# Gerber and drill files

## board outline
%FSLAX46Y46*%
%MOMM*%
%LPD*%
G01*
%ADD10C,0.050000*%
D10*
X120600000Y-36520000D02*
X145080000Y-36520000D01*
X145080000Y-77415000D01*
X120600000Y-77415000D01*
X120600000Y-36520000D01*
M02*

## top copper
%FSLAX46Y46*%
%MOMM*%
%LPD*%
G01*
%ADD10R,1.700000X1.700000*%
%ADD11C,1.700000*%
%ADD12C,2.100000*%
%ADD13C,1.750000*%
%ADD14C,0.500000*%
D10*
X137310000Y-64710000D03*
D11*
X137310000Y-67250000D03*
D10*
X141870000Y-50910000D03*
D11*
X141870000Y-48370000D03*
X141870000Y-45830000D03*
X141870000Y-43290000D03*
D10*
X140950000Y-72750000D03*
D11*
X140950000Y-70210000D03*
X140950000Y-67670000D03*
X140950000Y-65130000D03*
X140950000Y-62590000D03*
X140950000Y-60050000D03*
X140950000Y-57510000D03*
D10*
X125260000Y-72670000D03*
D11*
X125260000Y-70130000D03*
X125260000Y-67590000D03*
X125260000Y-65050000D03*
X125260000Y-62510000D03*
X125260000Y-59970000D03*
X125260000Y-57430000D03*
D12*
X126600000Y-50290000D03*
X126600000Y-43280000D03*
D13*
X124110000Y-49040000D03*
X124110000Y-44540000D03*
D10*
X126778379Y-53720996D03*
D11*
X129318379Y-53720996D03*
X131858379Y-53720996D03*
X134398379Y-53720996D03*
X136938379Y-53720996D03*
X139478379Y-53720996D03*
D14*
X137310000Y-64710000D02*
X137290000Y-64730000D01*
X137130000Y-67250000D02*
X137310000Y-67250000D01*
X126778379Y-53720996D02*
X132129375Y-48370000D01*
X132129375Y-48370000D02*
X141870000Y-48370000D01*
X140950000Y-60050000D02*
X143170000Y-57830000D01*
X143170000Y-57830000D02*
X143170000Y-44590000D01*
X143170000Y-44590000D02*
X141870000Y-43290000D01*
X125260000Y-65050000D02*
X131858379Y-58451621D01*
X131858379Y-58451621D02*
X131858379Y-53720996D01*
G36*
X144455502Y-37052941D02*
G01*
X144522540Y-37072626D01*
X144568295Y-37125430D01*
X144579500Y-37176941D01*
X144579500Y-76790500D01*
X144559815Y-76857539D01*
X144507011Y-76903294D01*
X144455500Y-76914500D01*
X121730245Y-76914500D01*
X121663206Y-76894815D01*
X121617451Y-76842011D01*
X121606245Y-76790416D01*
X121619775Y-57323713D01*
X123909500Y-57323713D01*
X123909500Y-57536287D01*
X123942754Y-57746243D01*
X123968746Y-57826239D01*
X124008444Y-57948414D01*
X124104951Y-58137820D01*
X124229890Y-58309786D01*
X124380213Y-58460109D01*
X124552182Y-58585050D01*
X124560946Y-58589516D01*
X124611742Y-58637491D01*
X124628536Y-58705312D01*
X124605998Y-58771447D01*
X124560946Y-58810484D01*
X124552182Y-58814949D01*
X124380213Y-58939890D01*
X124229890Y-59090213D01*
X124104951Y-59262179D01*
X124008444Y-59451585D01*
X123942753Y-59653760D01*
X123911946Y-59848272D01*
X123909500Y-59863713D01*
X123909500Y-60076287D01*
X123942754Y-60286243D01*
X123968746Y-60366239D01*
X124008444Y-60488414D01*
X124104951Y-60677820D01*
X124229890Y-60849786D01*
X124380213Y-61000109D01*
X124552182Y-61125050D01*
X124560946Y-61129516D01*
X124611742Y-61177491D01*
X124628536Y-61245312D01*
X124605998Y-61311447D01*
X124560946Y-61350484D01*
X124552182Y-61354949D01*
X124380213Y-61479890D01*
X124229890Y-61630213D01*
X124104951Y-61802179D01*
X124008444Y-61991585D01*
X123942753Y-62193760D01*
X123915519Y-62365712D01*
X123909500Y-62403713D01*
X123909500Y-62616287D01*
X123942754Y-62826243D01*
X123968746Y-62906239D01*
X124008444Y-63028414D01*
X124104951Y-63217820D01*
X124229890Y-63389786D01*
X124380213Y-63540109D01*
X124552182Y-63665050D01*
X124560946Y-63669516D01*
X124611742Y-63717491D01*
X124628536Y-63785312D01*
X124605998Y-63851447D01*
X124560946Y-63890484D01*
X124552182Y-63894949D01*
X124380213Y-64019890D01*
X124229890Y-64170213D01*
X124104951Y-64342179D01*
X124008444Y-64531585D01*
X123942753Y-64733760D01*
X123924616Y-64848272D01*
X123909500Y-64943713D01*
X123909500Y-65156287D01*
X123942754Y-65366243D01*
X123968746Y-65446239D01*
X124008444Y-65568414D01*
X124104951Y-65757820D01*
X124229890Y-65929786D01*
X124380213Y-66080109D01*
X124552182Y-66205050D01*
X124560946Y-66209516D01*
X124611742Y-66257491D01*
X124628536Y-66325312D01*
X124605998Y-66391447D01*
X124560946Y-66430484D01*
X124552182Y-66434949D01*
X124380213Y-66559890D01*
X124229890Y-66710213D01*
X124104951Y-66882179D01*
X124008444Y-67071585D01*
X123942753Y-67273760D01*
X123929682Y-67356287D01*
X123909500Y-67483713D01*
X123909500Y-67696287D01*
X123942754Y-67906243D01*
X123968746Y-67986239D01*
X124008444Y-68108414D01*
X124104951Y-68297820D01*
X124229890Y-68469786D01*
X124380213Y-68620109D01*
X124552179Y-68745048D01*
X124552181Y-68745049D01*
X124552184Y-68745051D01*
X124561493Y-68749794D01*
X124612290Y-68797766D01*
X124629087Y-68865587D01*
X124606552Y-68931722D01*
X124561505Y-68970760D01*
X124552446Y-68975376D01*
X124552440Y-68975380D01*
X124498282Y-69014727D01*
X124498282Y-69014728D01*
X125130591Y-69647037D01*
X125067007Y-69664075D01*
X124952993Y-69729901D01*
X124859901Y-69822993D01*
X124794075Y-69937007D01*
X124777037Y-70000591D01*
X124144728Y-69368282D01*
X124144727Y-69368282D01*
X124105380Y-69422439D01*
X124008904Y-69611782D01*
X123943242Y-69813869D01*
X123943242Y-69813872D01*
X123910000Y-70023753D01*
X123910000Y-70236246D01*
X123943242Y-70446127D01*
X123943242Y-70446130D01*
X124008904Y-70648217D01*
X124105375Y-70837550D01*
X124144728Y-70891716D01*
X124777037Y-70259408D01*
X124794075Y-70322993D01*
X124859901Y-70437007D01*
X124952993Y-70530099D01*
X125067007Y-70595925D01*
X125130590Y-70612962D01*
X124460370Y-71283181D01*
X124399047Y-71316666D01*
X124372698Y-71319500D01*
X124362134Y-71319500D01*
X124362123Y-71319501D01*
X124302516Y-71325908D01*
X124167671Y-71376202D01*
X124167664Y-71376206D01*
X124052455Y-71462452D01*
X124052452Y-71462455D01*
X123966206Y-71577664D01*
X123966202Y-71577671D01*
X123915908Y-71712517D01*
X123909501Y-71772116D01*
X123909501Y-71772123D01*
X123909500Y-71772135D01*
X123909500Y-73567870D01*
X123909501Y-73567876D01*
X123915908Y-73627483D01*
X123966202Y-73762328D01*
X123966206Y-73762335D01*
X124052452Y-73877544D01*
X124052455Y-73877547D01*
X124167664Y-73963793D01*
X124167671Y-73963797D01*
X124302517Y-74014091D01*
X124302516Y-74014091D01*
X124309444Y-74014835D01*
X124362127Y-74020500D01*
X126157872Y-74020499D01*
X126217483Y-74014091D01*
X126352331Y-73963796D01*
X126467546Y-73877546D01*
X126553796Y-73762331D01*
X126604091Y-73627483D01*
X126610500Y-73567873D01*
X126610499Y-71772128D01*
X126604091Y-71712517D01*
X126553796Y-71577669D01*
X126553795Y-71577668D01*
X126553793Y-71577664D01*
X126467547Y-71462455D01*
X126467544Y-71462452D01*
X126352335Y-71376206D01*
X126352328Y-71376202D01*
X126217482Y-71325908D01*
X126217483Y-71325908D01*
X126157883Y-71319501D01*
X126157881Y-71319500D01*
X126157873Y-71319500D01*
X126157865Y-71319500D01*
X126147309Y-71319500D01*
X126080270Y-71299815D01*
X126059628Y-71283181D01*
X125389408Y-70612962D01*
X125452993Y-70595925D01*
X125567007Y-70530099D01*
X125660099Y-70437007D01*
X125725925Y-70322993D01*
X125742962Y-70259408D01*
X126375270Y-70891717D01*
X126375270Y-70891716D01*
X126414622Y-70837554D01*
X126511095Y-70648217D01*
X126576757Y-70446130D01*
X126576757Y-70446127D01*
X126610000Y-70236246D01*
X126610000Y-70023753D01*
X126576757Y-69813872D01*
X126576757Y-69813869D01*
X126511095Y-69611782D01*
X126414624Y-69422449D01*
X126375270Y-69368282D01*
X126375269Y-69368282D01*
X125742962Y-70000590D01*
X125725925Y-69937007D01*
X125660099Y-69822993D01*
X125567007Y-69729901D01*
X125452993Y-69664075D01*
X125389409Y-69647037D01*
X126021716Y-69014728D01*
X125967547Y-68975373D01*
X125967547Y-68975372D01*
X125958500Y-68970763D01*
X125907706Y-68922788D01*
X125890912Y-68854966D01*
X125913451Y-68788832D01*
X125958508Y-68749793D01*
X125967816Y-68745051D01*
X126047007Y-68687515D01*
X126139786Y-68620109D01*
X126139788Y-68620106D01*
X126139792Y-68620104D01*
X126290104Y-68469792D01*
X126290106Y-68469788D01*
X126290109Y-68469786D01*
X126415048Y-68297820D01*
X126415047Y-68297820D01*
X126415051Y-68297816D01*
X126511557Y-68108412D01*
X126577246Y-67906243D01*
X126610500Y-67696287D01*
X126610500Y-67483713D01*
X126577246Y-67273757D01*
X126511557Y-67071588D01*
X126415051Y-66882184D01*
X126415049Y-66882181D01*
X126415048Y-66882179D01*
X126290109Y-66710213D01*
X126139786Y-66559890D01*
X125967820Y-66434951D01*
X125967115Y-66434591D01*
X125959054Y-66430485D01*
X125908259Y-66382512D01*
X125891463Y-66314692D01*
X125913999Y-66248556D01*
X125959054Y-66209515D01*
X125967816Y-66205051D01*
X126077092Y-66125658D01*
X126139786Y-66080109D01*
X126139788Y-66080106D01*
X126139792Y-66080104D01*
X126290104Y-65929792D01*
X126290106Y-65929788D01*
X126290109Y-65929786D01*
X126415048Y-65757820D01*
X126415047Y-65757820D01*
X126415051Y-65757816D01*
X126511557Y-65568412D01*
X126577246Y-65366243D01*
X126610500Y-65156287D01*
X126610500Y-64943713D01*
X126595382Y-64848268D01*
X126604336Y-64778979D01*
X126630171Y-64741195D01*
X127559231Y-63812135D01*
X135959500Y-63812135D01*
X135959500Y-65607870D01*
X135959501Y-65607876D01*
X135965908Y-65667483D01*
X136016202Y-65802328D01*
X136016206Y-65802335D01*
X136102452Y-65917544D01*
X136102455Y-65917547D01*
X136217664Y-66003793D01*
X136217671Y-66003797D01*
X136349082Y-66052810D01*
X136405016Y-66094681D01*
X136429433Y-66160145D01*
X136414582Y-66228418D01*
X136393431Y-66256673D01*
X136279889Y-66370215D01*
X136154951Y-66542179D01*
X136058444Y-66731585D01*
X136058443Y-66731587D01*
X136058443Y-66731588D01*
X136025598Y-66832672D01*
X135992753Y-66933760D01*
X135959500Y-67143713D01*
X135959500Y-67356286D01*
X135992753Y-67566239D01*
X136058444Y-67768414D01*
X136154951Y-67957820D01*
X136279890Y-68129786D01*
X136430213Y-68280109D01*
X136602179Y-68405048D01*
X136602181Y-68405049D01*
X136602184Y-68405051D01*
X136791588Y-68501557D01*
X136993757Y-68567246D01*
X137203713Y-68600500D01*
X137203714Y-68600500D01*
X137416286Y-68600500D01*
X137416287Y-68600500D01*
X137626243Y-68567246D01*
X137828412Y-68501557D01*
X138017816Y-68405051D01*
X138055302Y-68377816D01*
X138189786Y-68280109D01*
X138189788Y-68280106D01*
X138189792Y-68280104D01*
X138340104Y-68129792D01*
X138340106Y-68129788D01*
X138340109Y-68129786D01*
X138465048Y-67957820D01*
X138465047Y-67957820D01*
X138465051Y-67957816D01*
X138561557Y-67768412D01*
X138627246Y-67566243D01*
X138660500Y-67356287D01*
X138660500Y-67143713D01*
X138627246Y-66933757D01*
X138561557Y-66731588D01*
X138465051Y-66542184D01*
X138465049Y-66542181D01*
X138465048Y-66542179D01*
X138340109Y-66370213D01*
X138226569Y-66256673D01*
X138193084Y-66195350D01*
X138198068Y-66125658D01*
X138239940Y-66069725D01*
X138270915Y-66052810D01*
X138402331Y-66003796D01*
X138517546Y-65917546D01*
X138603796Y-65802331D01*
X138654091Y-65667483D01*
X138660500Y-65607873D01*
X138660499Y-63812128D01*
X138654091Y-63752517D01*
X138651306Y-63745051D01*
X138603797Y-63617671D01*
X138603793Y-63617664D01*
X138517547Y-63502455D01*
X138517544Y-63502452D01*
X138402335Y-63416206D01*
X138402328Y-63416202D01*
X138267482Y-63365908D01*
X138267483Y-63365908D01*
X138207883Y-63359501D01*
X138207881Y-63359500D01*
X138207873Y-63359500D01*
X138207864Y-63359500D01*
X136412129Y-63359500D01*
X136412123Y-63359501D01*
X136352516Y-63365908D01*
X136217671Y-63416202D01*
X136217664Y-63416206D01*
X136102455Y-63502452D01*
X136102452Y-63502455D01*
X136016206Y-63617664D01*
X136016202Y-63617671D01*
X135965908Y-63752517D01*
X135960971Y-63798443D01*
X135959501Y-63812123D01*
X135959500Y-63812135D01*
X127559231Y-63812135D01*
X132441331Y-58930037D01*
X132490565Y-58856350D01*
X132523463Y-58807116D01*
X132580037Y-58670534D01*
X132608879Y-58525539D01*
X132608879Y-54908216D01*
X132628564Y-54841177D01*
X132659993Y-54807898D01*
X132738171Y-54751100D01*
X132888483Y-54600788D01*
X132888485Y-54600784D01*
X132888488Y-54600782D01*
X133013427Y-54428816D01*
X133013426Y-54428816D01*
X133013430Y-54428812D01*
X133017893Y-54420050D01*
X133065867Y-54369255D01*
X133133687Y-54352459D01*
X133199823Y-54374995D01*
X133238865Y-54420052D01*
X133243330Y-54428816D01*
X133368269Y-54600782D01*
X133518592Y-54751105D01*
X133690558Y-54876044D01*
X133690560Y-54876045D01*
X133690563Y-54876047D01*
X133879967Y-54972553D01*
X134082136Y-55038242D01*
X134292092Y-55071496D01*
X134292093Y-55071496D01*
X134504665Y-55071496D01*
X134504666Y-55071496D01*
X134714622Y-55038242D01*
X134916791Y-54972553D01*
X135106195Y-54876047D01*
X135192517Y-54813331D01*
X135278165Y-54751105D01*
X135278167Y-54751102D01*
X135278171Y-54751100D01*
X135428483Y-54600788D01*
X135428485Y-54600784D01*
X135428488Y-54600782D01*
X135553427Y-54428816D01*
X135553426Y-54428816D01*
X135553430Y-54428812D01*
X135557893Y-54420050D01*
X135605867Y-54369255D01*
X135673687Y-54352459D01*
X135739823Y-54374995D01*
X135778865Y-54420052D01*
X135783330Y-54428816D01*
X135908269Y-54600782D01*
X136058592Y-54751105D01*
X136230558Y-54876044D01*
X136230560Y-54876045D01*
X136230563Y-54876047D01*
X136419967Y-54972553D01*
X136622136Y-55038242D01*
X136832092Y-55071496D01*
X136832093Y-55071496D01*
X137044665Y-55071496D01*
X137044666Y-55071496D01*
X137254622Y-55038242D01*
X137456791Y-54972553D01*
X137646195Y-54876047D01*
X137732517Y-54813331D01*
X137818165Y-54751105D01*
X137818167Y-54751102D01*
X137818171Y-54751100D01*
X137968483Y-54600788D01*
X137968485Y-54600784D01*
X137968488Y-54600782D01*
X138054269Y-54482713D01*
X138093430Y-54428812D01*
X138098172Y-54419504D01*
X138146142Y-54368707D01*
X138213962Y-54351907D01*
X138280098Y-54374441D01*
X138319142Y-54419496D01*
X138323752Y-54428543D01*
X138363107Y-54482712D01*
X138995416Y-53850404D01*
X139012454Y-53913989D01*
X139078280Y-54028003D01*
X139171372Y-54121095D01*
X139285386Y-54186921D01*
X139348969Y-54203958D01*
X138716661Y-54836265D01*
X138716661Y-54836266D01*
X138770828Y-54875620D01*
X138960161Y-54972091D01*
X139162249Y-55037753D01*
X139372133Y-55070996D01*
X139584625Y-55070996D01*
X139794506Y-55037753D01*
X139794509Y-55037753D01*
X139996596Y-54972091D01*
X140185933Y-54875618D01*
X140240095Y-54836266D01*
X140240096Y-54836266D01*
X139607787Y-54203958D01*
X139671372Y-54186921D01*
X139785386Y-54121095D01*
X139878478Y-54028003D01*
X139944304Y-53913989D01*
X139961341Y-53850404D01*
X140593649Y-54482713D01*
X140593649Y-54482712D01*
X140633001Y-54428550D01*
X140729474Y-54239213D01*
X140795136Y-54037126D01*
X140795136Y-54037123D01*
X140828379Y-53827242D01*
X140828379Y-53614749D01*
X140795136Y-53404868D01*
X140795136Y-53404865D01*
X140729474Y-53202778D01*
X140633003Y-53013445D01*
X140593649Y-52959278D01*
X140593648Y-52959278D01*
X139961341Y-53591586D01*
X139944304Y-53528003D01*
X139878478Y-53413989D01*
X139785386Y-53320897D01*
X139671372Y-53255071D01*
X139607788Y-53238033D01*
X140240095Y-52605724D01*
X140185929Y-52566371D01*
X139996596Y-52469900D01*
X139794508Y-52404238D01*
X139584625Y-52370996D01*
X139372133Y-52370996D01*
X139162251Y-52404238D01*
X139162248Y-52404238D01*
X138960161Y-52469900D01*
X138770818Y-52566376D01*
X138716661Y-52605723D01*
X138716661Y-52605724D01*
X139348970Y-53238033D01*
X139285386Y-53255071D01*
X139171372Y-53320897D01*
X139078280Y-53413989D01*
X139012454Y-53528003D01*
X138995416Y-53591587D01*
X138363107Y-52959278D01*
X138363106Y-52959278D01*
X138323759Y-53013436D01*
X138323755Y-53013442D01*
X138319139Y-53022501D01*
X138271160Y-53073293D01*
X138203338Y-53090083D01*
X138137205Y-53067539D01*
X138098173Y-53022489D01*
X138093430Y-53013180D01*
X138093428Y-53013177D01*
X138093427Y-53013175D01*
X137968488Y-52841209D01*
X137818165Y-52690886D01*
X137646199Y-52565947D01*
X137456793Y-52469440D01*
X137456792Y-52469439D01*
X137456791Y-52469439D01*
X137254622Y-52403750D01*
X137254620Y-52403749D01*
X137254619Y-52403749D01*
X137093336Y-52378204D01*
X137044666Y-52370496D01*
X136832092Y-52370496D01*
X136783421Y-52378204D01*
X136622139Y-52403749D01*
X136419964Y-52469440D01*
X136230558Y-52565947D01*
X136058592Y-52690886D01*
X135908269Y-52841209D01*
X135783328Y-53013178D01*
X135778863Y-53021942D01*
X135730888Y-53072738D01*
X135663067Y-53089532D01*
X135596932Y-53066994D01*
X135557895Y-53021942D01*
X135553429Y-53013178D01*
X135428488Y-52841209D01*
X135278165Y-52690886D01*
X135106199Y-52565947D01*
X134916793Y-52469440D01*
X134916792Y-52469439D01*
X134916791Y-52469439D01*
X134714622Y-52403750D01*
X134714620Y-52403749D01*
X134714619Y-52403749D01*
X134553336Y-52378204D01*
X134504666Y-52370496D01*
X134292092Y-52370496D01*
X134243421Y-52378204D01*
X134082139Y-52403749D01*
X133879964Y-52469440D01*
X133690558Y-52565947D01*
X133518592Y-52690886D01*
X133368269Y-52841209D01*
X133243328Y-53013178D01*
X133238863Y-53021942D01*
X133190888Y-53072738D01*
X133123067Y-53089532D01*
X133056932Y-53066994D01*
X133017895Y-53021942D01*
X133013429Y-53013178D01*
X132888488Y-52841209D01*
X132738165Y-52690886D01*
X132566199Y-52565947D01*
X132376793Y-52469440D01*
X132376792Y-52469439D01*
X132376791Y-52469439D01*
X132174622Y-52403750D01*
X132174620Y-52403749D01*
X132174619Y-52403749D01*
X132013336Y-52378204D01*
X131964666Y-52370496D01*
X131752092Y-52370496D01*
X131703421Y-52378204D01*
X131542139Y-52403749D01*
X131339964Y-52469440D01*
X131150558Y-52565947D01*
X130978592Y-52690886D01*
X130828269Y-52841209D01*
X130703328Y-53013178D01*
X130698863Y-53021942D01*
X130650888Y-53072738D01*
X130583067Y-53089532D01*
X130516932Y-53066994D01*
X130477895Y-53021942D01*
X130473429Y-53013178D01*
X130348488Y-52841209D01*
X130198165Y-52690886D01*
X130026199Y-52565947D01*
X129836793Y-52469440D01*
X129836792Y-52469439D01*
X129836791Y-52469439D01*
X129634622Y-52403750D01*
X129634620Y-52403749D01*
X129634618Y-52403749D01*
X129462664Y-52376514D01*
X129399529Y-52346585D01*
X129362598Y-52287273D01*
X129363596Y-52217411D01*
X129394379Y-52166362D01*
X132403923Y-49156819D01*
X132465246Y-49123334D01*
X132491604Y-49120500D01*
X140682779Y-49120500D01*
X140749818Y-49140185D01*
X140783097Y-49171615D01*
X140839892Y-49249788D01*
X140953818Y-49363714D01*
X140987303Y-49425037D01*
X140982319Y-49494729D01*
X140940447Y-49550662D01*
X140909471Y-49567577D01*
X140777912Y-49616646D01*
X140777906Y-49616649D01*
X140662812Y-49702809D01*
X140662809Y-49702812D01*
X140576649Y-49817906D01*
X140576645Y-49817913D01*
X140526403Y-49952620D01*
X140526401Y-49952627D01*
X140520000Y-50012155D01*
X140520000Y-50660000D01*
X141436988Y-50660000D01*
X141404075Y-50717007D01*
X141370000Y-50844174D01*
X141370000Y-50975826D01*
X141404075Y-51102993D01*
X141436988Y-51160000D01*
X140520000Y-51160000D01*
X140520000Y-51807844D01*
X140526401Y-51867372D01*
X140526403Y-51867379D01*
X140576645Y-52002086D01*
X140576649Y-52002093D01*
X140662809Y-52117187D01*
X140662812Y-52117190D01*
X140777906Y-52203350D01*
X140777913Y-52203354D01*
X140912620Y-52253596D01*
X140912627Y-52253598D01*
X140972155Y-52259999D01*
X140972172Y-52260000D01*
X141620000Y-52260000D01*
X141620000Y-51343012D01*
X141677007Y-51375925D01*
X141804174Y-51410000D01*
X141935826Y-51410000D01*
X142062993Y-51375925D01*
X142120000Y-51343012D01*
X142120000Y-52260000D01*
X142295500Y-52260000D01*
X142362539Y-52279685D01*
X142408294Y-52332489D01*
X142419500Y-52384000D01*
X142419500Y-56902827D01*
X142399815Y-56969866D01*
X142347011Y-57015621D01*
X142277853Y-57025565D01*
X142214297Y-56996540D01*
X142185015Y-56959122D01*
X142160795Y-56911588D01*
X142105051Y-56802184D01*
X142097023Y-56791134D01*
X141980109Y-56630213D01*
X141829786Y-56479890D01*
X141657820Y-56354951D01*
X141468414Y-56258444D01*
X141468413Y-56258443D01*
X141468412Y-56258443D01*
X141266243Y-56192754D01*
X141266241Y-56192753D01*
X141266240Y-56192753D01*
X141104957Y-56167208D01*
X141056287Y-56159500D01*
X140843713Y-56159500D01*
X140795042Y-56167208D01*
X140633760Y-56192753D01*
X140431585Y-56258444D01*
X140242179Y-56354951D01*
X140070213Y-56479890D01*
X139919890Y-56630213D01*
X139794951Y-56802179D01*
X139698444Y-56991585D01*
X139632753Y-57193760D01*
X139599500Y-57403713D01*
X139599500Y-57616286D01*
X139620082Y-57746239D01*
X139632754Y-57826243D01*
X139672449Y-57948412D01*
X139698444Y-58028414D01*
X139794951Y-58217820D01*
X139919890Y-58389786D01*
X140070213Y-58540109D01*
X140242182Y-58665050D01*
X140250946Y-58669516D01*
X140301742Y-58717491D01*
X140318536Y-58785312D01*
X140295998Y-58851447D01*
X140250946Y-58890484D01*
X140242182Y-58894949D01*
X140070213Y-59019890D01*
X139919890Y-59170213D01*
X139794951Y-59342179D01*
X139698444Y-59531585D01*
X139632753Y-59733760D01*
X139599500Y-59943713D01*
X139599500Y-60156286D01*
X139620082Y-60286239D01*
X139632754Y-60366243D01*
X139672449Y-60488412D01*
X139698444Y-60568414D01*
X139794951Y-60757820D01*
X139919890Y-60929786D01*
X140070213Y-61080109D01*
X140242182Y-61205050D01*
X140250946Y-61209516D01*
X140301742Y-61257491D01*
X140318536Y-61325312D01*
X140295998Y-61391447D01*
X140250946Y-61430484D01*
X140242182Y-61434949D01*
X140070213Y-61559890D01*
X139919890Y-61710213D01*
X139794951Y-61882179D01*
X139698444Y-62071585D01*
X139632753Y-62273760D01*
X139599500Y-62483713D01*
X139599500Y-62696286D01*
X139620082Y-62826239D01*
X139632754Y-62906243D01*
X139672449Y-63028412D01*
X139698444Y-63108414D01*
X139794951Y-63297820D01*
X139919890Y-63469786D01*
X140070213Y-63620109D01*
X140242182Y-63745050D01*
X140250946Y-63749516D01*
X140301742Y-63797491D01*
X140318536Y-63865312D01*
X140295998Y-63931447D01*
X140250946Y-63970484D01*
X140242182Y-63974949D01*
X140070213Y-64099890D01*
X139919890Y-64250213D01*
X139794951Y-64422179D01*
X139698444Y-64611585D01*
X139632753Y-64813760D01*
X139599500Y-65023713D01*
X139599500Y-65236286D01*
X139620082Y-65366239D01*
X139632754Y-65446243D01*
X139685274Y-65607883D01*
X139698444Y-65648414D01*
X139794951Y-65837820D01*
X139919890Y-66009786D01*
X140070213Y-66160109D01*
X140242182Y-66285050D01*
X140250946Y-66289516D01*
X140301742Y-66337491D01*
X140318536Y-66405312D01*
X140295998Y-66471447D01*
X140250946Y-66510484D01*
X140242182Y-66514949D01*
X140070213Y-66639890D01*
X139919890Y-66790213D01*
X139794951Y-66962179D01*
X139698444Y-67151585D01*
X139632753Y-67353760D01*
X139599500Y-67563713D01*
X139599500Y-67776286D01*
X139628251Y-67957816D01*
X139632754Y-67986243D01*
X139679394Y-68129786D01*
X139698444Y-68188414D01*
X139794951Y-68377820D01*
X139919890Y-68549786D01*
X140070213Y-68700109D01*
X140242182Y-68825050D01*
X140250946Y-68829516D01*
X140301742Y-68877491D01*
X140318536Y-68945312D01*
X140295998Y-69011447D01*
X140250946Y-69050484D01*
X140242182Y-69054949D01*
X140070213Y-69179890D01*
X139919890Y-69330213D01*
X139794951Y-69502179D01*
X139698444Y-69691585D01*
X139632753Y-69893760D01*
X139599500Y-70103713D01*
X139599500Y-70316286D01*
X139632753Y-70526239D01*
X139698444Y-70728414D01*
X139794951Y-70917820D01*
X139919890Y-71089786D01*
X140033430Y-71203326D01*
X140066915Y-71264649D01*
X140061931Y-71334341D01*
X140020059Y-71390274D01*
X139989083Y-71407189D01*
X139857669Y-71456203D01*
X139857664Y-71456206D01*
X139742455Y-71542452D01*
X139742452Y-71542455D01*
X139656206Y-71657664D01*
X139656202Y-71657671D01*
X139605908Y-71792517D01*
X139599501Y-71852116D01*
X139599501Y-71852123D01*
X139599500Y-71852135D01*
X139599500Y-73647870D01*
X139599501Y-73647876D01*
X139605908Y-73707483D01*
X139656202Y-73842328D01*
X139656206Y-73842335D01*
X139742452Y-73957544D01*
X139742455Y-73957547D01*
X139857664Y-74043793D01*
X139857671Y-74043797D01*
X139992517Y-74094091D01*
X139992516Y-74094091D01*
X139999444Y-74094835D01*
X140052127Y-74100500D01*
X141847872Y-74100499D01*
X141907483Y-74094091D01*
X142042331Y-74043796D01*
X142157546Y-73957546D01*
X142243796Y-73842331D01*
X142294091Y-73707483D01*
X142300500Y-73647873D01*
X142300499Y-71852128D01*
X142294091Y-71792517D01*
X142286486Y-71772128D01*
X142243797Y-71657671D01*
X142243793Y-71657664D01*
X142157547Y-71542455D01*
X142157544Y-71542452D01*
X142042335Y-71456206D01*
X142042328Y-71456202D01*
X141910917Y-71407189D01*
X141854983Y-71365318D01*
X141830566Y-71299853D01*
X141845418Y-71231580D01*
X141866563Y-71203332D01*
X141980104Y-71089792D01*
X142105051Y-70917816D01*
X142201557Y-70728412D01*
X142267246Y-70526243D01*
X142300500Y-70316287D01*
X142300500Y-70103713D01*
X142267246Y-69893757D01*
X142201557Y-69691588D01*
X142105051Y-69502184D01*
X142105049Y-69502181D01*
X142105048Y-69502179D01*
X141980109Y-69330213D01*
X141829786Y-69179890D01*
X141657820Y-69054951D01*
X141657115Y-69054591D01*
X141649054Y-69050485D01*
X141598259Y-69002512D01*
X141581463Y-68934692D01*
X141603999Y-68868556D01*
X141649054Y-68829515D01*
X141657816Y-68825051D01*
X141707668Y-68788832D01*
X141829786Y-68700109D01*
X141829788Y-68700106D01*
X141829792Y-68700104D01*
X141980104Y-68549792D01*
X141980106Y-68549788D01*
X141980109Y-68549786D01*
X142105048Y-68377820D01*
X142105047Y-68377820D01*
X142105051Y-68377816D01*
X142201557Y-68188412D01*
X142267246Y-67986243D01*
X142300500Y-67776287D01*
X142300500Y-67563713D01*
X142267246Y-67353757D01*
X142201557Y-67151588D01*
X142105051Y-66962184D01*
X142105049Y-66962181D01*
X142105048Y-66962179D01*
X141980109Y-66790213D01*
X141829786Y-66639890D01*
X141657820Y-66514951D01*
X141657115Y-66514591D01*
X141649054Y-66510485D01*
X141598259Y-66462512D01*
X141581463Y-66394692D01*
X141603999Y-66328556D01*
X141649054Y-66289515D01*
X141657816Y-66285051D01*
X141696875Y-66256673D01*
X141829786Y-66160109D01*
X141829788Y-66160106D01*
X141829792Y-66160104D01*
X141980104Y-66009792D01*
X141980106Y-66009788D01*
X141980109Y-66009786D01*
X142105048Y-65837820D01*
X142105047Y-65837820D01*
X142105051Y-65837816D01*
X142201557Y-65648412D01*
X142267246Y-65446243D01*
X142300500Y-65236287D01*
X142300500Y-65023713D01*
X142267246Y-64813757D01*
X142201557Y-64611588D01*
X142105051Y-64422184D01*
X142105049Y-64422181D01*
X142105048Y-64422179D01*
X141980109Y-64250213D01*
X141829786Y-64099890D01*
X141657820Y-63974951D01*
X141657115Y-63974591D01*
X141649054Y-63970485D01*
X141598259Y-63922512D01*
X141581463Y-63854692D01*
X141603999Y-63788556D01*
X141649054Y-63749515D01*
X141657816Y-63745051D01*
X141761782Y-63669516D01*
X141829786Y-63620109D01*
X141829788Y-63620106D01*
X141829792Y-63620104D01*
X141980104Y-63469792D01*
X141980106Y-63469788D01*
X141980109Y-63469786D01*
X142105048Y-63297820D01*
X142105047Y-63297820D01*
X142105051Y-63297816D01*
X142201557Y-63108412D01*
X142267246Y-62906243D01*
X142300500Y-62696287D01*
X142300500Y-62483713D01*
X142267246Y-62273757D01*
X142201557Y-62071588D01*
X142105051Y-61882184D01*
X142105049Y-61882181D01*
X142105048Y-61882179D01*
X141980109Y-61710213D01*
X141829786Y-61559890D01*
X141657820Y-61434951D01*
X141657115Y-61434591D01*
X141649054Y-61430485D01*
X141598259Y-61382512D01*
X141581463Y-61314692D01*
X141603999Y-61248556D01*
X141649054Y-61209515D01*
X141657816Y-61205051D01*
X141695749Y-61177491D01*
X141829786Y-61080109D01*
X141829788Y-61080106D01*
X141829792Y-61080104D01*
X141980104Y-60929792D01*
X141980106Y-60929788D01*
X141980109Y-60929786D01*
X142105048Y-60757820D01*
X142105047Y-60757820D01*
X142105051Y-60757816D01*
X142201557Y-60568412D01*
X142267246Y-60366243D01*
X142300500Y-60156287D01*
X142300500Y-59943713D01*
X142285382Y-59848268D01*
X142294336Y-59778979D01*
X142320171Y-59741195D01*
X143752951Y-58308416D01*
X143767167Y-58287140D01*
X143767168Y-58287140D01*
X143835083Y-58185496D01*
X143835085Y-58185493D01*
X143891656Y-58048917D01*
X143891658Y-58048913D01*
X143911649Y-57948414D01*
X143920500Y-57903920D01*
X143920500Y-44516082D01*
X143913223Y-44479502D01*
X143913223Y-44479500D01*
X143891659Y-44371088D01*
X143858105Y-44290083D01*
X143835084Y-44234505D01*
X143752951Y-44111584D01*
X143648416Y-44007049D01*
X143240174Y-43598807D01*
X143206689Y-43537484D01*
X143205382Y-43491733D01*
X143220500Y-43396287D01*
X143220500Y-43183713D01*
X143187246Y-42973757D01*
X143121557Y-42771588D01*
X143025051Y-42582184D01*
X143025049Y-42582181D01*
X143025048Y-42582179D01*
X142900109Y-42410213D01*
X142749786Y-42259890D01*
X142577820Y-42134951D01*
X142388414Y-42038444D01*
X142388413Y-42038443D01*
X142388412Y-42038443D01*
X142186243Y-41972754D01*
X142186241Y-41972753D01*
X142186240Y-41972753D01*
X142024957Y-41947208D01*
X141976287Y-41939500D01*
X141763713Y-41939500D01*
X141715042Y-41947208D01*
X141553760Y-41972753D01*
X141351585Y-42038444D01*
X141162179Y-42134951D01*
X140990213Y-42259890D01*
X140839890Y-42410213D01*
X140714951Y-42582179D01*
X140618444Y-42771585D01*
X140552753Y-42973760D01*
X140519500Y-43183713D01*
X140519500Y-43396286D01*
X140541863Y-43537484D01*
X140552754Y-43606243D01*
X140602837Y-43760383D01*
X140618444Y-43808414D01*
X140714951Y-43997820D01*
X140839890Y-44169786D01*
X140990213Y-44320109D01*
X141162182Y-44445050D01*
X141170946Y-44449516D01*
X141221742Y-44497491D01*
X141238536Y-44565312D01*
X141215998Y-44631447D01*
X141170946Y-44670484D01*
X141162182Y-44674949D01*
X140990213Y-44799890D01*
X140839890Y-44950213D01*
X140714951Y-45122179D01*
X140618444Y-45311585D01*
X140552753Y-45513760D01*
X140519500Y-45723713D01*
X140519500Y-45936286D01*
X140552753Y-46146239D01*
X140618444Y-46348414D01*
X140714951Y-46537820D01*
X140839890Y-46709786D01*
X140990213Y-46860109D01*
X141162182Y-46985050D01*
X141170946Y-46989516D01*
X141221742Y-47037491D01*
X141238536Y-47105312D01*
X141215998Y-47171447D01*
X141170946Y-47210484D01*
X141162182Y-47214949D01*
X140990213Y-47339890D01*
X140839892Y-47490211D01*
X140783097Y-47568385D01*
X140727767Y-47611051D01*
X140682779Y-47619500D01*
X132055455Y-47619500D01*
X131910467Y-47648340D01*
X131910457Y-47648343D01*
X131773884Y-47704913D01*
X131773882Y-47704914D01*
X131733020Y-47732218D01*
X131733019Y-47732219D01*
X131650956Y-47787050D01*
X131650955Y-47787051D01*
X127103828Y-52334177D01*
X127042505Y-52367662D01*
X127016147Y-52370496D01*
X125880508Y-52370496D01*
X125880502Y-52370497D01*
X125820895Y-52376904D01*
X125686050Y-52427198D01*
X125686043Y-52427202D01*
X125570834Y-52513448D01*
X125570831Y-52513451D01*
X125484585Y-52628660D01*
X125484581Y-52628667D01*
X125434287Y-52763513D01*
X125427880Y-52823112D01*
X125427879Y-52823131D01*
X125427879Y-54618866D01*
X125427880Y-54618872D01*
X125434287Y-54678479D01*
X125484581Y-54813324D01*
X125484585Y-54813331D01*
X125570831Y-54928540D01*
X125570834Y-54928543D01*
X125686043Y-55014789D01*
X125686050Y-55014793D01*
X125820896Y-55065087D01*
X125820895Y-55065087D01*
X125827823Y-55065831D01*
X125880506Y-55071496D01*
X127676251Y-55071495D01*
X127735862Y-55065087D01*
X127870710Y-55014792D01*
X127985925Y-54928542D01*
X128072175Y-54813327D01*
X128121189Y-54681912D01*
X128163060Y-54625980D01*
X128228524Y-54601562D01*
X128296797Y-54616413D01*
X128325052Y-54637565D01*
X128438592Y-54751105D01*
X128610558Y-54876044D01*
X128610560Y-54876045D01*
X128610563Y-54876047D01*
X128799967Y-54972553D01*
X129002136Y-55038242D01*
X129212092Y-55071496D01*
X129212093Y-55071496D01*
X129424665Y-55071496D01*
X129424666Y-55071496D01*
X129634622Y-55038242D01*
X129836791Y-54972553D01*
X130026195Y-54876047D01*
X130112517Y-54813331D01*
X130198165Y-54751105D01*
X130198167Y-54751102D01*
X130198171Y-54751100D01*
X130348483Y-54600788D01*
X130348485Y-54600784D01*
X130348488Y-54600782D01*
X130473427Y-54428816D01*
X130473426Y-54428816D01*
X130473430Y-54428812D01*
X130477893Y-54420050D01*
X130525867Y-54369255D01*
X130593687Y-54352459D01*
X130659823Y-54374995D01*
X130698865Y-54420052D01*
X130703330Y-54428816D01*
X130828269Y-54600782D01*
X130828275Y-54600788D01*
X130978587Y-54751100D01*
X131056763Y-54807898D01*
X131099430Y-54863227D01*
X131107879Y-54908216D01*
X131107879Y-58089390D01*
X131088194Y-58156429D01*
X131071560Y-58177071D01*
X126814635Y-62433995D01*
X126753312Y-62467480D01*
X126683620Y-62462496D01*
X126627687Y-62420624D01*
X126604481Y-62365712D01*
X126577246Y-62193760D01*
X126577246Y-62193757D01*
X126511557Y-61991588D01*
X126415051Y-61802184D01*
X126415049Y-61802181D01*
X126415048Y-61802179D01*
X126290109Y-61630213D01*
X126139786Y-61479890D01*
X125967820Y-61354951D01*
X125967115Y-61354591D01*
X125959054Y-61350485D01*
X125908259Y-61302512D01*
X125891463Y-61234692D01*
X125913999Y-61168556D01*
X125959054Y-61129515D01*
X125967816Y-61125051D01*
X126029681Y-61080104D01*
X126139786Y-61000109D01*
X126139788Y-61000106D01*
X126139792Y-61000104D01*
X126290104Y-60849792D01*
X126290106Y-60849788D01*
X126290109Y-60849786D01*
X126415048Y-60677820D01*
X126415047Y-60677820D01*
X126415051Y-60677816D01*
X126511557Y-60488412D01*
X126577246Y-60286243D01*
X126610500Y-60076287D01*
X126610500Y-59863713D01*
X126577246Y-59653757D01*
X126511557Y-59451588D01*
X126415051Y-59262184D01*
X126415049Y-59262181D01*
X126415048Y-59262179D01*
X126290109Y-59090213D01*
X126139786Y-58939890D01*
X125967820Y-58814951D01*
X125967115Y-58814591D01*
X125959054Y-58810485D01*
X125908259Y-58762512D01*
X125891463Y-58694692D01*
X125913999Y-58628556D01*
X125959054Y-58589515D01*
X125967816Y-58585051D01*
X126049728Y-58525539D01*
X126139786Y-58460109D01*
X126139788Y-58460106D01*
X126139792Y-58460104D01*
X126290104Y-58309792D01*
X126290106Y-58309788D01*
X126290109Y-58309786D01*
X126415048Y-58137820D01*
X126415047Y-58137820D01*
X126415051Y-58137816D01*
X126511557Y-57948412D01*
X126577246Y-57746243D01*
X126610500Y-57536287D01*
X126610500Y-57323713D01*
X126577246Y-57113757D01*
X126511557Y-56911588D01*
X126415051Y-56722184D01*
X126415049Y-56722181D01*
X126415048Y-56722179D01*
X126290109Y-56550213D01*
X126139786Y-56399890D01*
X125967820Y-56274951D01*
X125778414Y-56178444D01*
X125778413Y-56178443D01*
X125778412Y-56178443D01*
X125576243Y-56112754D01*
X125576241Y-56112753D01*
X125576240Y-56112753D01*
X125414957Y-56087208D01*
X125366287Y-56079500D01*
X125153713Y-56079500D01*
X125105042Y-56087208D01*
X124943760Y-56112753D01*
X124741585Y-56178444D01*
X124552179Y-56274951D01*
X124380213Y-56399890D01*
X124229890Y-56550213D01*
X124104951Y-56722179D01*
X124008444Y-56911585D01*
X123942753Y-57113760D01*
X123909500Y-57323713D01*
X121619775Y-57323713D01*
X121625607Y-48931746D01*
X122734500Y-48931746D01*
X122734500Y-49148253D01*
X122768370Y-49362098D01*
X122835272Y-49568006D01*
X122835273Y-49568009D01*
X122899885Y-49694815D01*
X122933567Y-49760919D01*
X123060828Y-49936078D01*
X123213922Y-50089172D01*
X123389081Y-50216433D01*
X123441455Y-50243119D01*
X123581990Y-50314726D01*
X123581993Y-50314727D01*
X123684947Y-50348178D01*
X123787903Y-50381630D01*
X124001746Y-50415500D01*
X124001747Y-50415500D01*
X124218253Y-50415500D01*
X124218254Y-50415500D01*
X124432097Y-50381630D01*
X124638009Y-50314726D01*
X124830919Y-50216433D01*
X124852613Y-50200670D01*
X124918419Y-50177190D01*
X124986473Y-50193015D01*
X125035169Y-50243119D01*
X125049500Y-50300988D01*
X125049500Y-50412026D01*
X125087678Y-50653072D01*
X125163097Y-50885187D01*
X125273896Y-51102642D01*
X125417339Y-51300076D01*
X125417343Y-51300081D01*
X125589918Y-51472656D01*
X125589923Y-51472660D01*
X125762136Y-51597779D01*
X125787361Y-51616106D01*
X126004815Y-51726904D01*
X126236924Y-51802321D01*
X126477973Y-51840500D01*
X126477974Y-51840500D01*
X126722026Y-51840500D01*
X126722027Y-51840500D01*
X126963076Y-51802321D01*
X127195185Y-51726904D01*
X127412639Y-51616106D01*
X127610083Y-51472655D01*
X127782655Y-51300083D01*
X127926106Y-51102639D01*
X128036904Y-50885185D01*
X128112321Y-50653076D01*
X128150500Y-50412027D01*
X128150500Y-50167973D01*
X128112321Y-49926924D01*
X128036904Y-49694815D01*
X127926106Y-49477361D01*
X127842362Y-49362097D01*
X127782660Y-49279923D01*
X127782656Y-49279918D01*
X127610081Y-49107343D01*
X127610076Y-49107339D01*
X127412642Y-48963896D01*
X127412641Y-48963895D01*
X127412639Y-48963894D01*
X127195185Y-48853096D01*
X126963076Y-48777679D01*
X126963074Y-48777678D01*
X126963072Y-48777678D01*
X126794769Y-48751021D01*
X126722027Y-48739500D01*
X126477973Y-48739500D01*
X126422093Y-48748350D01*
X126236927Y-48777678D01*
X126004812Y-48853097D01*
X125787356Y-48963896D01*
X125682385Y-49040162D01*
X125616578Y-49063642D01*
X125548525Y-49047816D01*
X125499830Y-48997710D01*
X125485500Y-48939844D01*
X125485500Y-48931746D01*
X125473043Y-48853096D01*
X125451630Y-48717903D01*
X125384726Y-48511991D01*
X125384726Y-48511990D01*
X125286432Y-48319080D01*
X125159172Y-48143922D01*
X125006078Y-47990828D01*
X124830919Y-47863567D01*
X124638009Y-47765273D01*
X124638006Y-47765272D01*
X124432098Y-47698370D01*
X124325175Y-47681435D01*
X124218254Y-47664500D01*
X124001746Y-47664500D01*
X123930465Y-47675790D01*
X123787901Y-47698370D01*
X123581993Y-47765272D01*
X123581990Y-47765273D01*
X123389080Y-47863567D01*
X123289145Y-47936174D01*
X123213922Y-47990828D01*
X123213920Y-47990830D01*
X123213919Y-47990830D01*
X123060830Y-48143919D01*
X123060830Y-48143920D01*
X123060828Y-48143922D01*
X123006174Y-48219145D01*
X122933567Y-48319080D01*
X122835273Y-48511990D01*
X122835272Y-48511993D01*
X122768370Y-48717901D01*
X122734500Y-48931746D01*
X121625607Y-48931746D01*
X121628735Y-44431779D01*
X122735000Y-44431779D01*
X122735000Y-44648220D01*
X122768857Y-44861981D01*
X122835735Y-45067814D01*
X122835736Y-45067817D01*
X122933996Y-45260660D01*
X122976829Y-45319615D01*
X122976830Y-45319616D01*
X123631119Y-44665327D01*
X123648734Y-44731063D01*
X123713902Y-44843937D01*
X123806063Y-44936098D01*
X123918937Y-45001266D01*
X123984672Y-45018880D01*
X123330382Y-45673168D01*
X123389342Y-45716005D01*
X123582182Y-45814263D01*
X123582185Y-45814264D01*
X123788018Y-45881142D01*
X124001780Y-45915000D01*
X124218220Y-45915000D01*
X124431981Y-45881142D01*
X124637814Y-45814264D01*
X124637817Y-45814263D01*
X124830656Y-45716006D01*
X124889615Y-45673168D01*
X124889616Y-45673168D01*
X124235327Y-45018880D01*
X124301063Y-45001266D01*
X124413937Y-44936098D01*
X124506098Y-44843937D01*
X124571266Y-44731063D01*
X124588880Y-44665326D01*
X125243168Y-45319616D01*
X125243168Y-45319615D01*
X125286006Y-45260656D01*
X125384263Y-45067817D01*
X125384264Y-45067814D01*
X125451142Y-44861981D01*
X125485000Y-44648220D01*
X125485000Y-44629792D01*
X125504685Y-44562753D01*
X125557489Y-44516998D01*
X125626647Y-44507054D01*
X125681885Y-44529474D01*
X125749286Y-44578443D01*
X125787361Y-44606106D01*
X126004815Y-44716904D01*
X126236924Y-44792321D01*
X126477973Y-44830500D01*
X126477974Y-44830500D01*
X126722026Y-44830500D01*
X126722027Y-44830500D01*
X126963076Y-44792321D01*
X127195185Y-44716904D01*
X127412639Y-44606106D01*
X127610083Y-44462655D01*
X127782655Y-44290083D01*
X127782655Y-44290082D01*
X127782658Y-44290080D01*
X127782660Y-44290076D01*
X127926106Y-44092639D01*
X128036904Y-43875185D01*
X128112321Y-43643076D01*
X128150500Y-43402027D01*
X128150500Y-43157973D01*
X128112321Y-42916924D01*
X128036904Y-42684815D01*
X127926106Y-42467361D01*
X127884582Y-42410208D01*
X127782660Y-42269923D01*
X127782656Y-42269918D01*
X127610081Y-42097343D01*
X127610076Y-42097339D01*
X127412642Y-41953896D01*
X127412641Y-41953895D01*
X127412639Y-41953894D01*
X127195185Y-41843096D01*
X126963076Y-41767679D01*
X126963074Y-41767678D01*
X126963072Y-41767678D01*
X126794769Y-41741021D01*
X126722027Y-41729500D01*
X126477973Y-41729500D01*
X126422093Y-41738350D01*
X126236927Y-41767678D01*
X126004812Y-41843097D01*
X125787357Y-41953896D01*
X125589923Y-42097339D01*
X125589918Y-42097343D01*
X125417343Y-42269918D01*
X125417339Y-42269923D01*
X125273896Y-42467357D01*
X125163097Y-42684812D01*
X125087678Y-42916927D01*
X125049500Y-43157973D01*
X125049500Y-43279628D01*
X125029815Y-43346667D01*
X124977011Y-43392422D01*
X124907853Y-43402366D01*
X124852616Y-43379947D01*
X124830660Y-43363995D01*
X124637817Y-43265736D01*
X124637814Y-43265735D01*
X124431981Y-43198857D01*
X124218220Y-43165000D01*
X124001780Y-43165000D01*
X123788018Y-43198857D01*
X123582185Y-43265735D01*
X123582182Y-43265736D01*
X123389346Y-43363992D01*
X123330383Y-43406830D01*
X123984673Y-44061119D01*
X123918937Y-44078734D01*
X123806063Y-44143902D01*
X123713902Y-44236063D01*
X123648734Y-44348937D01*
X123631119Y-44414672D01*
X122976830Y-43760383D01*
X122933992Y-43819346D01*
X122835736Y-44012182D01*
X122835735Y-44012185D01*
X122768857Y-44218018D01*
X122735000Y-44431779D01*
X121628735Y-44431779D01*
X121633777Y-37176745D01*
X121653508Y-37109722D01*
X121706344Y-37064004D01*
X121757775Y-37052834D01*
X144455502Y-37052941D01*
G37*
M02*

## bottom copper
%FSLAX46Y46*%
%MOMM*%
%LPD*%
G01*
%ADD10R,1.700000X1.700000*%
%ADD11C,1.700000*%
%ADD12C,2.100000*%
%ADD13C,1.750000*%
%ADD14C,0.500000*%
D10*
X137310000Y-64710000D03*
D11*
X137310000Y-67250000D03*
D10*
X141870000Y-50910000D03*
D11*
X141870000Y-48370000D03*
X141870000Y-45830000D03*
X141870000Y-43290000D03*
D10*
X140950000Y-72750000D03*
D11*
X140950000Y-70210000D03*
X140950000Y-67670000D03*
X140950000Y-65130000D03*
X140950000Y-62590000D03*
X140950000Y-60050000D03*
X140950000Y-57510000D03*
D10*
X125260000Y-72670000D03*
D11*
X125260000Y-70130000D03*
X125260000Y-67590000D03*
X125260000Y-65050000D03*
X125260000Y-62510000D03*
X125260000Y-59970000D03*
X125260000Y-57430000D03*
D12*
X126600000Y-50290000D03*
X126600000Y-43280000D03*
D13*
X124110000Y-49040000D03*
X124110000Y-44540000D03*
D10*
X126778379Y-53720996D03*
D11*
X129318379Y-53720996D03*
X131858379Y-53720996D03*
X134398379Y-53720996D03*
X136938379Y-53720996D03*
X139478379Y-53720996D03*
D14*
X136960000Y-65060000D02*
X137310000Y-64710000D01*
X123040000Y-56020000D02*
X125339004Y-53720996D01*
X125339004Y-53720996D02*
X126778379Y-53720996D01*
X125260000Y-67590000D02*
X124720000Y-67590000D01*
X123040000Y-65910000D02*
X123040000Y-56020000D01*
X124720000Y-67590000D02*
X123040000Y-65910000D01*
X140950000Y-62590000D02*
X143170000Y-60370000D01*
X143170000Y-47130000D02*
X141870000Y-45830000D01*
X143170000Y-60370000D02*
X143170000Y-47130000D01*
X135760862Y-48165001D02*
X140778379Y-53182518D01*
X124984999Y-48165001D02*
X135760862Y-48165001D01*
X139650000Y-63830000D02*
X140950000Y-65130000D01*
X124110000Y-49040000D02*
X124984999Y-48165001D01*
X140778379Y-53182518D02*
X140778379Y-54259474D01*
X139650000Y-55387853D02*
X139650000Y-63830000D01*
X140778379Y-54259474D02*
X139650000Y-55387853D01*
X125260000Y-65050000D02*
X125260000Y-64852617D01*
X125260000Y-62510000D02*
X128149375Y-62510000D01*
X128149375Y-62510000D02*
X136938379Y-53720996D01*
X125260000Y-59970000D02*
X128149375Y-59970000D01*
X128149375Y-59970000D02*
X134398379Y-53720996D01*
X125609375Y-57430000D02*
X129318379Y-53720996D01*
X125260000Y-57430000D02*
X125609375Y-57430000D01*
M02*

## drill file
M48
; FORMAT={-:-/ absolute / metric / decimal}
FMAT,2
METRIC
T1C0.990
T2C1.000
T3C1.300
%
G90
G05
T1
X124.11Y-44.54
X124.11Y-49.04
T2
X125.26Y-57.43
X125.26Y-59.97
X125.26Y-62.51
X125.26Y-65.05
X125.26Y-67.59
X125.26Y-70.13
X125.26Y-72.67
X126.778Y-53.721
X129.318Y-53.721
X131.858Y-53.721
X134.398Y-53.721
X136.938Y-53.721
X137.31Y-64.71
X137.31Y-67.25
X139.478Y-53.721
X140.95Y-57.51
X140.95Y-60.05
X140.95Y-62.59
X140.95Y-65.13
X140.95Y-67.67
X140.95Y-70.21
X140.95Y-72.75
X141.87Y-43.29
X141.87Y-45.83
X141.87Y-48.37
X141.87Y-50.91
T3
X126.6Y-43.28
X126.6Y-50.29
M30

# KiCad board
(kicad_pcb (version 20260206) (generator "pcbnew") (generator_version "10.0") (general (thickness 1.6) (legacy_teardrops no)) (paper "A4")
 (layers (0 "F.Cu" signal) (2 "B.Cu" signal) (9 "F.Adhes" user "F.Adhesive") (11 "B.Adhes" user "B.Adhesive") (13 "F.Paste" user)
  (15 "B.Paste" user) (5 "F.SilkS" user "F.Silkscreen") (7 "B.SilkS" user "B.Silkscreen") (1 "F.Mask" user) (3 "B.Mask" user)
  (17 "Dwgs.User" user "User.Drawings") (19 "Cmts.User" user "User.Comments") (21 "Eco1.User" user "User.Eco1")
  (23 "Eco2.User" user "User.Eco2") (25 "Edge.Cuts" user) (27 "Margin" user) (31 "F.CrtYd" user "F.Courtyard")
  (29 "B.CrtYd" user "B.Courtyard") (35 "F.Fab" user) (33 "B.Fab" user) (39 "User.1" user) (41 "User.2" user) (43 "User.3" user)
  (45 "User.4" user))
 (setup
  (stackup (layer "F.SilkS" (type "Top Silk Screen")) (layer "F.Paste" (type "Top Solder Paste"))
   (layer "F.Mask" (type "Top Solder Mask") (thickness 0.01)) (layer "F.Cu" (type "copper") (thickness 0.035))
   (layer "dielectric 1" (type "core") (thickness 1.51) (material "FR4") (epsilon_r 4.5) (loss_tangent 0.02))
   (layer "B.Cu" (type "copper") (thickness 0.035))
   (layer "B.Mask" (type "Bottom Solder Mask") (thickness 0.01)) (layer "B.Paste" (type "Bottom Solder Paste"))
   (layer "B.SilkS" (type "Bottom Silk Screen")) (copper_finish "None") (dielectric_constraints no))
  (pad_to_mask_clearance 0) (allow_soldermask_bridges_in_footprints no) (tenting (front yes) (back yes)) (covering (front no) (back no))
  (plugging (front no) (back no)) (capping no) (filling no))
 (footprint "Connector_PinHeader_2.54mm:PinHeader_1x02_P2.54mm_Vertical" (layer "F.Cu") (at 137.31 64.71)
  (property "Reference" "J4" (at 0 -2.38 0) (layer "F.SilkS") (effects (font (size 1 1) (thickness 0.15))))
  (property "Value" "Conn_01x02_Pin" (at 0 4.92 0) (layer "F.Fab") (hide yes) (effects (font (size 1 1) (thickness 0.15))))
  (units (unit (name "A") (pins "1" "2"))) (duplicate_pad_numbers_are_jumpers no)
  (pad "1" thru_hole rect (at 0 0) (size 1.7 1.7) (drill 1) (layers "*.Cu" "*.Mask") (remove_unused_layers no) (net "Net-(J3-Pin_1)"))
  (pad "2" thru_hole circle (at 0 2.54) (size 1.7 1.7) (drill 1) (layers "*.Cu" "*.Mask") (remove_unused_layers no) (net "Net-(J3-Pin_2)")))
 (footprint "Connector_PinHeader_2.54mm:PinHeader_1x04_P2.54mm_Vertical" (layer "F.Cu") (at 141.87 50.91 180)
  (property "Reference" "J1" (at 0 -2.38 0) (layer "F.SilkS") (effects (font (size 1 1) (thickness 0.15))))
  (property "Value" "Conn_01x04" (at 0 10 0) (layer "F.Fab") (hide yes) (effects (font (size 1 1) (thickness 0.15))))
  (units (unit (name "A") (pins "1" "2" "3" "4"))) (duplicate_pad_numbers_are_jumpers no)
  (pad "1" thru_hole rect (at 0 0 180) (size 1.7 1.7) (drill 1) (layers "*.Cu" "*.Mask") (remove_unused_layers no) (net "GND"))
  (pad "2" thru_hole circle (at 0 2.54 180) (size 1.7 1.7) (drill 1) (layers "*.Cu" "*.Mask") (remove_unused_layers no) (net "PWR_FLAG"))
  (pad "3" thru_hole circle (at 0 5.08 180) (size 1.7 1.7) (drill 1) (layers "*.Cu" "*.Mask") (remove_unused_layers no)
   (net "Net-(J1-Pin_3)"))
  (pad "4" thru_hole circle (at 0 7.62 180) (size 1.7 1.7) (drill 1) (layers "*.Cu" "*.Mask") (remove_unused_layers no)
   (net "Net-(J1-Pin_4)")))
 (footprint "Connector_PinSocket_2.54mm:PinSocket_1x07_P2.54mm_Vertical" (layer "F.Cu") (at 140.95 72.75 180)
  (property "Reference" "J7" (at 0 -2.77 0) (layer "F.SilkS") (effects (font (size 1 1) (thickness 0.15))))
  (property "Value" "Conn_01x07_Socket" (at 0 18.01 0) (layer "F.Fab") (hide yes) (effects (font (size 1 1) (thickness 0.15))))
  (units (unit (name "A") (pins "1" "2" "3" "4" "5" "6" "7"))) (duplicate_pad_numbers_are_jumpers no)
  (pad "1" thru_hole rect (at 0 0 180) (size 1.7 1.7) (drill 1) (layers "*.Cu" "*.Mask") (remove_unused_layers no) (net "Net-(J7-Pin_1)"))
  (pad "2" thru_hole circle (at 0 2.54 180) (size 1.7 1.7) (drill 1) (layers "*.Cu" "*.Mask") (remove_unused_layers no)
   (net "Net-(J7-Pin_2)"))
  (pad "3" thru_hole circle (at 0 5.08 180) (size 1.7 1.7) (drill 1) (layers "*.Cu" "*.Mask") (remove_unused_layers no)
   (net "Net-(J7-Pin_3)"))
  (pad "4" thru_hole circle (at 0 7.62 180) (size 1.7 1.7) (drill 1) (layers "*.Cu" "*.Mask") (remove_unused_layers no)
   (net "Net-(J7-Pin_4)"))
  (pad "5" thru_hole circle (at 0 10.16 180) (size 1.7 1.7) (drill 1) (layers "*.Cu" "*.Mask") (remove_unused_layers no)
   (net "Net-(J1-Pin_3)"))
  (pad "6" thru_hole circle (at 0 12.7 180) (size 1.7 1.7) (drill 1) (layers "*.Cu" "*.Mask") (remove_unused_layers no)
   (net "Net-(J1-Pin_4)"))
  (pad "7" thru_hole circle (at 0 15.24 180) (size 1.7 1.7) (drill 1) (layers "*.Cu" "*.Mask") (remove_unused_layers no)
   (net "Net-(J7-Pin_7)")))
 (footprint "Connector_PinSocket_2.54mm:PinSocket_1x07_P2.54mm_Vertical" (layer "F.Cu") (at 125.26 72.67 180)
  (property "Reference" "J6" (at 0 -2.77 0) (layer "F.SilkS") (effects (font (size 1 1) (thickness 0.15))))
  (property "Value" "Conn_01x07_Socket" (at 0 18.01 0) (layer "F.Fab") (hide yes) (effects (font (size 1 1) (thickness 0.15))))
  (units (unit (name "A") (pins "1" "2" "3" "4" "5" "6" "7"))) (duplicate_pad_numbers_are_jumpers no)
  (pad "1" thru_hole rect (at 0 0 180) (size 1.7 1.7) (drill 1) (layers "*.Cu" "*.Mask") (remove_unused_layers no) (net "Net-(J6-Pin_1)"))
  (pad "2" thru_hole circle (at 0 2.54 180) (size 1.7 1.7) (drill 1) (layers "*.Cu" "*.Mask") (remove_unused_layers no) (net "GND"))
  (pad "3" thru_hole circle (at 0 5.08 180) (size 1.7 1.7) (drill 1) (layers "*.Cu" "*.Mask") (remove_unused_layers no) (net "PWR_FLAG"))
  (pad "4" thru_hole circle (at 0 7.62 180) (size 1.7 1.7) (drill 1) (layers "*.Cu" "*.Mask") (remove_unused_layers no)
   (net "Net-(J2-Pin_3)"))
  (pad "5" thru_hole circle (at 0 10.16 180) (size 1.7 1.7) (drill 1) (layers "*.Cu" "*.Mask") (remove_unused_layers no)
   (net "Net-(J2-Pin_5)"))
  (pad "6" thru_hole circle (at 0 12.7 180) (size 1.7 1.7) (drill 1) (layers "*.Cu" "*.Mask") (remove_unused_layers no)
   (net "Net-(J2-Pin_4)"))
  (pad "7" thru_hole circle (at 0 15.24 180) (size 1.7 1.7) (drill 1) (layers "*.Cu" "*.Mask") (remove_unused_layers no)
   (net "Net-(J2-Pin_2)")))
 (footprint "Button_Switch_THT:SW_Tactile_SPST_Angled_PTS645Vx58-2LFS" (layer "F.Cu") (at 124.11 49.04 90)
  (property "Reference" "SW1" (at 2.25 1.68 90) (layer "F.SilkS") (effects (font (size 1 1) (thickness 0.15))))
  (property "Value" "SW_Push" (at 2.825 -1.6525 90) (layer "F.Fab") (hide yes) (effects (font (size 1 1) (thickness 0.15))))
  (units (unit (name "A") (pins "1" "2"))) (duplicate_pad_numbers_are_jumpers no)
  (pad "" thru_hole circle (at -1.25 2.49 90) (size 2.1 2.1) (drill 1.3) (layers "*.Cu" "*.Mask") (remove_unused_layers no))
  (pad "" thru_hole circle (at 5.76 2.49 90) (size 2.1 2.1) (drill 1.3) (layers "*.Cu" "*.Mask") (remove_unused_layers no))
  (pad "1" thru_hole circle (at 0 0 90) (size 1.75 1.75) (drill 0.99) (layers "*.Cu" "*.Mask") (remove_unused_layers no)
   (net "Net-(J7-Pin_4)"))
  (pad "2" thru_hole circle (at 4.5 0 90) (size 1.75 1.75) (drill 0.99) (layers "*.Cu" "*.Mask") (remove_unused_layers no) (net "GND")))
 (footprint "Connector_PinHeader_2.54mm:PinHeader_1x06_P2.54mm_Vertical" (layer "B.Cu") (at 126.778379 53.720996 -90)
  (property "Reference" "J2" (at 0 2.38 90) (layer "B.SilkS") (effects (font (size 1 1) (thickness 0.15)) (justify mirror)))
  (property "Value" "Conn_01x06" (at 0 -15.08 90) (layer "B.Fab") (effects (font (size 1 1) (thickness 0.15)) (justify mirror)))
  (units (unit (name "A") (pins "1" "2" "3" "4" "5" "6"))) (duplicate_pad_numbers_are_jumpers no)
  (pad "1" thru_hole rect (at 0 0 270) (size 1.7 1.7) (drill 1) (layers "*.Cu" "*.Mask") (remove_unused_layers no) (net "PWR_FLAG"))
  (pad "2" thru_hole circle (at 0 -2.54 270) (size 1.7 1.7) (drill 1) (layers "*.Cu" "*.Mask") (remove_unused_layers no)
   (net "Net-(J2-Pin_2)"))
  (pad "3" thru_hole circle (at 0 -5.08 270) (size 1.7 1.7) (drill 1) (layers "*.Cu" "*.Mask") (remove_unused_layers no)
   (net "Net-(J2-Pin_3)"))
  (pad "4" thru_hole circle (at 0 -7.62 270) (size 1.7 1.7) (drill 1) (layers "*.Cu" "*.Mask") (remove_unused_layers no)
   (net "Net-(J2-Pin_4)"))
  (pad "5" thru_hole circle (at 0 -10.16 270) (size 1.7 1.7) (drill 1) (layers "*.Cu" "*.Mask") (remove_unused_layers no)
   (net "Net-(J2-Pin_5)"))
  (pad "6" thru_hole circle (at 0 -12.7 270) (size 1.7 1.7) (drill 1) (layers "*.Cu" "*.Mask") (remove_unused_layers no) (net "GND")))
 (gr_rect (start 120.6 36.52) (end 145.08 77.415) (stroke (width 0.05) (type default)) (fill no) (layer "Edge.Cuts"))
 (segment (start 137.31 64.71) (end 137.29 64.73) (width 0.5) (layer "F.Cu") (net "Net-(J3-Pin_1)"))
 (segment (start 136.96 65.06) (end 137.31 64.71) (width 0.5) (layer "B.Cu") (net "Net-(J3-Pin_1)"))
 (segment (start 137.13 67.25) (end 137.31 67.25) (width 0.5) (layer "F.Cu") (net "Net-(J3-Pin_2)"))
 (segment (start 126.778379 53.720996) (end 132.129375 48.37) (width 0.5) (layer "F.Cu") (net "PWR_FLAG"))
 (segment (start 132.129375 48.37) (end 141.87 48.37) (width 0.5) (layer "F.Cu") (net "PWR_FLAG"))
 (segment (start 123.04 56.02) (end 125.339004 53.720996) (width 0.5) (layer "B.Cu") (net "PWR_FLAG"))
 (segment (start 125.339004 53.720996) (end 126.778379 53.720996) (width 0.5) (layer "B.Cu") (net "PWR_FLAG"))
 (segment (start 125.26 67.59) (end 124.72 67.59) (width 0.5) (layer "B.Cu") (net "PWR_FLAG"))
 (segment (start 123.04 65.91) (end 123.04 56.02) (width 0.5) (layer "B.Cu") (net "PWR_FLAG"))
 (segment (start 124.72 67.59) (end 123.04 65.91) (width 0.5) (layer "B.Cu") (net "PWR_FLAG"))
 (segment (start 140.95 62.59) (end 143.17 60.37) (width 0.5) (layer "B.Cu") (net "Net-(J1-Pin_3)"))
 (segment (start 143.17 47.13) (end 141.87 45.83) (width 0.5) (layer "B.Cu") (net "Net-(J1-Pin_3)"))
 (segment (start 143.17 60.37) (end 143.17 47.13) (width 0.5) (layer "B.Cu") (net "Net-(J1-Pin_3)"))
 (segment (start 140.95 60.05) (end 143.17 57.83) (width 0.5) (layer "F.Cu") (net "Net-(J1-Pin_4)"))
 (segment (start 143.17 57.83) (end 143.17 44.59) (width 0.5) (layer "F.Cu") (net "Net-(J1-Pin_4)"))
 (segment (start 143.17 44.59) (end 141.87 43.29) (width 0.5) (layer "F.Cu") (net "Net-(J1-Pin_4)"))
 (segment (start 135.760862 48.165001) (end 140.778379 53.182518) (width 0.5) (layer "B.Cu") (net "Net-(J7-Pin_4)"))
 (segment (start 124.984999 48.165001) (end 135.760862 48.165001) (width 0.5) (layer "B.Cu") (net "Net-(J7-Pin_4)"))
 (segment (start 139.65 63.83) (end 140.95 65.13) (width 0.5) (layer "B.Cu") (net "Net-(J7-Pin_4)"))
 (segment (start 124.11 49.04) (end 124.984999 48.165001) (width 0.5) (layer "B.Cu") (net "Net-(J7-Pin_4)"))
 (segment (start 140.778379 53.182518) (end 140.778379 54.259474) (width 0.5) (layer "B.Cu") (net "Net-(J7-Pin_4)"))
 (segment (start 139.65 55.387853) (end 139.65 63.83) (width 0.5) (layer "B.Cu") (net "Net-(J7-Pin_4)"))
 (segment (start 140.778379 54.259474) (end 139.65 55.387853) (width 0.5) (layer "B.Cu") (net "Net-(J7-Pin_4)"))
 (segment (start 125.26 65.05) (end 131.858379 58.451621) (width 0.5) (layer "F.Cu") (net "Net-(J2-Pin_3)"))
 (segment (start 131.858379 58.451621) (end 131.858379 53.720996) (width 0.5) (layer "F.Cu") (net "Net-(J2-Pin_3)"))
 (segment (start 125.26 65.05) (end 125.26 64.852617) (width 0.5) (layer "B.Cu") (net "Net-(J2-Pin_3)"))
 (segment (start 125.26 62.51) (end 128.149375 62.51) (width 0.5) (layer "B.Cu") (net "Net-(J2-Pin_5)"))
 (segment (start 128.149375 62.51) (end 136.938379 53.720996) (width 0.5) (layer "B.Cu") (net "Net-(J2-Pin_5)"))
 (segment (start 125.26 59.97) (end 128.149375 59.97) (width 0.5) (layer "B.Cu") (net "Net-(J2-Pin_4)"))
 (segment (start 128.149375 59.97) (end 134.398379 53.720996) (width 0.5) (layer "B.Cu") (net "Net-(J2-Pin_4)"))
 (segment (start 125.609375 57.43) (end 129.318379 53.720996) (width 0.5) (layer "B.Cu") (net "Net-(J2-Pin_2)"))
 (segment (start 125.26 57.43) (end 125.609375 57.43) (width 0.5) (layer "B.Cu") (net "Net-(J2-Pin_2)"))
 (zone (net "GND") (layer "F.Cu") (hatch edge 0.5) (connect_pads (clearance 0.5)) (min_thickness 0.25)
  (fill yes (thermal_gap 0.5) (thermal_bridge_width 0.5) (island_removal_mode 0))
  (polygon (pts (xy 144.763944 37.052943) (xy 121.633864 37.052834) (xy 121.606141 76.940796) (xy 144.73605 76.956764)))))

